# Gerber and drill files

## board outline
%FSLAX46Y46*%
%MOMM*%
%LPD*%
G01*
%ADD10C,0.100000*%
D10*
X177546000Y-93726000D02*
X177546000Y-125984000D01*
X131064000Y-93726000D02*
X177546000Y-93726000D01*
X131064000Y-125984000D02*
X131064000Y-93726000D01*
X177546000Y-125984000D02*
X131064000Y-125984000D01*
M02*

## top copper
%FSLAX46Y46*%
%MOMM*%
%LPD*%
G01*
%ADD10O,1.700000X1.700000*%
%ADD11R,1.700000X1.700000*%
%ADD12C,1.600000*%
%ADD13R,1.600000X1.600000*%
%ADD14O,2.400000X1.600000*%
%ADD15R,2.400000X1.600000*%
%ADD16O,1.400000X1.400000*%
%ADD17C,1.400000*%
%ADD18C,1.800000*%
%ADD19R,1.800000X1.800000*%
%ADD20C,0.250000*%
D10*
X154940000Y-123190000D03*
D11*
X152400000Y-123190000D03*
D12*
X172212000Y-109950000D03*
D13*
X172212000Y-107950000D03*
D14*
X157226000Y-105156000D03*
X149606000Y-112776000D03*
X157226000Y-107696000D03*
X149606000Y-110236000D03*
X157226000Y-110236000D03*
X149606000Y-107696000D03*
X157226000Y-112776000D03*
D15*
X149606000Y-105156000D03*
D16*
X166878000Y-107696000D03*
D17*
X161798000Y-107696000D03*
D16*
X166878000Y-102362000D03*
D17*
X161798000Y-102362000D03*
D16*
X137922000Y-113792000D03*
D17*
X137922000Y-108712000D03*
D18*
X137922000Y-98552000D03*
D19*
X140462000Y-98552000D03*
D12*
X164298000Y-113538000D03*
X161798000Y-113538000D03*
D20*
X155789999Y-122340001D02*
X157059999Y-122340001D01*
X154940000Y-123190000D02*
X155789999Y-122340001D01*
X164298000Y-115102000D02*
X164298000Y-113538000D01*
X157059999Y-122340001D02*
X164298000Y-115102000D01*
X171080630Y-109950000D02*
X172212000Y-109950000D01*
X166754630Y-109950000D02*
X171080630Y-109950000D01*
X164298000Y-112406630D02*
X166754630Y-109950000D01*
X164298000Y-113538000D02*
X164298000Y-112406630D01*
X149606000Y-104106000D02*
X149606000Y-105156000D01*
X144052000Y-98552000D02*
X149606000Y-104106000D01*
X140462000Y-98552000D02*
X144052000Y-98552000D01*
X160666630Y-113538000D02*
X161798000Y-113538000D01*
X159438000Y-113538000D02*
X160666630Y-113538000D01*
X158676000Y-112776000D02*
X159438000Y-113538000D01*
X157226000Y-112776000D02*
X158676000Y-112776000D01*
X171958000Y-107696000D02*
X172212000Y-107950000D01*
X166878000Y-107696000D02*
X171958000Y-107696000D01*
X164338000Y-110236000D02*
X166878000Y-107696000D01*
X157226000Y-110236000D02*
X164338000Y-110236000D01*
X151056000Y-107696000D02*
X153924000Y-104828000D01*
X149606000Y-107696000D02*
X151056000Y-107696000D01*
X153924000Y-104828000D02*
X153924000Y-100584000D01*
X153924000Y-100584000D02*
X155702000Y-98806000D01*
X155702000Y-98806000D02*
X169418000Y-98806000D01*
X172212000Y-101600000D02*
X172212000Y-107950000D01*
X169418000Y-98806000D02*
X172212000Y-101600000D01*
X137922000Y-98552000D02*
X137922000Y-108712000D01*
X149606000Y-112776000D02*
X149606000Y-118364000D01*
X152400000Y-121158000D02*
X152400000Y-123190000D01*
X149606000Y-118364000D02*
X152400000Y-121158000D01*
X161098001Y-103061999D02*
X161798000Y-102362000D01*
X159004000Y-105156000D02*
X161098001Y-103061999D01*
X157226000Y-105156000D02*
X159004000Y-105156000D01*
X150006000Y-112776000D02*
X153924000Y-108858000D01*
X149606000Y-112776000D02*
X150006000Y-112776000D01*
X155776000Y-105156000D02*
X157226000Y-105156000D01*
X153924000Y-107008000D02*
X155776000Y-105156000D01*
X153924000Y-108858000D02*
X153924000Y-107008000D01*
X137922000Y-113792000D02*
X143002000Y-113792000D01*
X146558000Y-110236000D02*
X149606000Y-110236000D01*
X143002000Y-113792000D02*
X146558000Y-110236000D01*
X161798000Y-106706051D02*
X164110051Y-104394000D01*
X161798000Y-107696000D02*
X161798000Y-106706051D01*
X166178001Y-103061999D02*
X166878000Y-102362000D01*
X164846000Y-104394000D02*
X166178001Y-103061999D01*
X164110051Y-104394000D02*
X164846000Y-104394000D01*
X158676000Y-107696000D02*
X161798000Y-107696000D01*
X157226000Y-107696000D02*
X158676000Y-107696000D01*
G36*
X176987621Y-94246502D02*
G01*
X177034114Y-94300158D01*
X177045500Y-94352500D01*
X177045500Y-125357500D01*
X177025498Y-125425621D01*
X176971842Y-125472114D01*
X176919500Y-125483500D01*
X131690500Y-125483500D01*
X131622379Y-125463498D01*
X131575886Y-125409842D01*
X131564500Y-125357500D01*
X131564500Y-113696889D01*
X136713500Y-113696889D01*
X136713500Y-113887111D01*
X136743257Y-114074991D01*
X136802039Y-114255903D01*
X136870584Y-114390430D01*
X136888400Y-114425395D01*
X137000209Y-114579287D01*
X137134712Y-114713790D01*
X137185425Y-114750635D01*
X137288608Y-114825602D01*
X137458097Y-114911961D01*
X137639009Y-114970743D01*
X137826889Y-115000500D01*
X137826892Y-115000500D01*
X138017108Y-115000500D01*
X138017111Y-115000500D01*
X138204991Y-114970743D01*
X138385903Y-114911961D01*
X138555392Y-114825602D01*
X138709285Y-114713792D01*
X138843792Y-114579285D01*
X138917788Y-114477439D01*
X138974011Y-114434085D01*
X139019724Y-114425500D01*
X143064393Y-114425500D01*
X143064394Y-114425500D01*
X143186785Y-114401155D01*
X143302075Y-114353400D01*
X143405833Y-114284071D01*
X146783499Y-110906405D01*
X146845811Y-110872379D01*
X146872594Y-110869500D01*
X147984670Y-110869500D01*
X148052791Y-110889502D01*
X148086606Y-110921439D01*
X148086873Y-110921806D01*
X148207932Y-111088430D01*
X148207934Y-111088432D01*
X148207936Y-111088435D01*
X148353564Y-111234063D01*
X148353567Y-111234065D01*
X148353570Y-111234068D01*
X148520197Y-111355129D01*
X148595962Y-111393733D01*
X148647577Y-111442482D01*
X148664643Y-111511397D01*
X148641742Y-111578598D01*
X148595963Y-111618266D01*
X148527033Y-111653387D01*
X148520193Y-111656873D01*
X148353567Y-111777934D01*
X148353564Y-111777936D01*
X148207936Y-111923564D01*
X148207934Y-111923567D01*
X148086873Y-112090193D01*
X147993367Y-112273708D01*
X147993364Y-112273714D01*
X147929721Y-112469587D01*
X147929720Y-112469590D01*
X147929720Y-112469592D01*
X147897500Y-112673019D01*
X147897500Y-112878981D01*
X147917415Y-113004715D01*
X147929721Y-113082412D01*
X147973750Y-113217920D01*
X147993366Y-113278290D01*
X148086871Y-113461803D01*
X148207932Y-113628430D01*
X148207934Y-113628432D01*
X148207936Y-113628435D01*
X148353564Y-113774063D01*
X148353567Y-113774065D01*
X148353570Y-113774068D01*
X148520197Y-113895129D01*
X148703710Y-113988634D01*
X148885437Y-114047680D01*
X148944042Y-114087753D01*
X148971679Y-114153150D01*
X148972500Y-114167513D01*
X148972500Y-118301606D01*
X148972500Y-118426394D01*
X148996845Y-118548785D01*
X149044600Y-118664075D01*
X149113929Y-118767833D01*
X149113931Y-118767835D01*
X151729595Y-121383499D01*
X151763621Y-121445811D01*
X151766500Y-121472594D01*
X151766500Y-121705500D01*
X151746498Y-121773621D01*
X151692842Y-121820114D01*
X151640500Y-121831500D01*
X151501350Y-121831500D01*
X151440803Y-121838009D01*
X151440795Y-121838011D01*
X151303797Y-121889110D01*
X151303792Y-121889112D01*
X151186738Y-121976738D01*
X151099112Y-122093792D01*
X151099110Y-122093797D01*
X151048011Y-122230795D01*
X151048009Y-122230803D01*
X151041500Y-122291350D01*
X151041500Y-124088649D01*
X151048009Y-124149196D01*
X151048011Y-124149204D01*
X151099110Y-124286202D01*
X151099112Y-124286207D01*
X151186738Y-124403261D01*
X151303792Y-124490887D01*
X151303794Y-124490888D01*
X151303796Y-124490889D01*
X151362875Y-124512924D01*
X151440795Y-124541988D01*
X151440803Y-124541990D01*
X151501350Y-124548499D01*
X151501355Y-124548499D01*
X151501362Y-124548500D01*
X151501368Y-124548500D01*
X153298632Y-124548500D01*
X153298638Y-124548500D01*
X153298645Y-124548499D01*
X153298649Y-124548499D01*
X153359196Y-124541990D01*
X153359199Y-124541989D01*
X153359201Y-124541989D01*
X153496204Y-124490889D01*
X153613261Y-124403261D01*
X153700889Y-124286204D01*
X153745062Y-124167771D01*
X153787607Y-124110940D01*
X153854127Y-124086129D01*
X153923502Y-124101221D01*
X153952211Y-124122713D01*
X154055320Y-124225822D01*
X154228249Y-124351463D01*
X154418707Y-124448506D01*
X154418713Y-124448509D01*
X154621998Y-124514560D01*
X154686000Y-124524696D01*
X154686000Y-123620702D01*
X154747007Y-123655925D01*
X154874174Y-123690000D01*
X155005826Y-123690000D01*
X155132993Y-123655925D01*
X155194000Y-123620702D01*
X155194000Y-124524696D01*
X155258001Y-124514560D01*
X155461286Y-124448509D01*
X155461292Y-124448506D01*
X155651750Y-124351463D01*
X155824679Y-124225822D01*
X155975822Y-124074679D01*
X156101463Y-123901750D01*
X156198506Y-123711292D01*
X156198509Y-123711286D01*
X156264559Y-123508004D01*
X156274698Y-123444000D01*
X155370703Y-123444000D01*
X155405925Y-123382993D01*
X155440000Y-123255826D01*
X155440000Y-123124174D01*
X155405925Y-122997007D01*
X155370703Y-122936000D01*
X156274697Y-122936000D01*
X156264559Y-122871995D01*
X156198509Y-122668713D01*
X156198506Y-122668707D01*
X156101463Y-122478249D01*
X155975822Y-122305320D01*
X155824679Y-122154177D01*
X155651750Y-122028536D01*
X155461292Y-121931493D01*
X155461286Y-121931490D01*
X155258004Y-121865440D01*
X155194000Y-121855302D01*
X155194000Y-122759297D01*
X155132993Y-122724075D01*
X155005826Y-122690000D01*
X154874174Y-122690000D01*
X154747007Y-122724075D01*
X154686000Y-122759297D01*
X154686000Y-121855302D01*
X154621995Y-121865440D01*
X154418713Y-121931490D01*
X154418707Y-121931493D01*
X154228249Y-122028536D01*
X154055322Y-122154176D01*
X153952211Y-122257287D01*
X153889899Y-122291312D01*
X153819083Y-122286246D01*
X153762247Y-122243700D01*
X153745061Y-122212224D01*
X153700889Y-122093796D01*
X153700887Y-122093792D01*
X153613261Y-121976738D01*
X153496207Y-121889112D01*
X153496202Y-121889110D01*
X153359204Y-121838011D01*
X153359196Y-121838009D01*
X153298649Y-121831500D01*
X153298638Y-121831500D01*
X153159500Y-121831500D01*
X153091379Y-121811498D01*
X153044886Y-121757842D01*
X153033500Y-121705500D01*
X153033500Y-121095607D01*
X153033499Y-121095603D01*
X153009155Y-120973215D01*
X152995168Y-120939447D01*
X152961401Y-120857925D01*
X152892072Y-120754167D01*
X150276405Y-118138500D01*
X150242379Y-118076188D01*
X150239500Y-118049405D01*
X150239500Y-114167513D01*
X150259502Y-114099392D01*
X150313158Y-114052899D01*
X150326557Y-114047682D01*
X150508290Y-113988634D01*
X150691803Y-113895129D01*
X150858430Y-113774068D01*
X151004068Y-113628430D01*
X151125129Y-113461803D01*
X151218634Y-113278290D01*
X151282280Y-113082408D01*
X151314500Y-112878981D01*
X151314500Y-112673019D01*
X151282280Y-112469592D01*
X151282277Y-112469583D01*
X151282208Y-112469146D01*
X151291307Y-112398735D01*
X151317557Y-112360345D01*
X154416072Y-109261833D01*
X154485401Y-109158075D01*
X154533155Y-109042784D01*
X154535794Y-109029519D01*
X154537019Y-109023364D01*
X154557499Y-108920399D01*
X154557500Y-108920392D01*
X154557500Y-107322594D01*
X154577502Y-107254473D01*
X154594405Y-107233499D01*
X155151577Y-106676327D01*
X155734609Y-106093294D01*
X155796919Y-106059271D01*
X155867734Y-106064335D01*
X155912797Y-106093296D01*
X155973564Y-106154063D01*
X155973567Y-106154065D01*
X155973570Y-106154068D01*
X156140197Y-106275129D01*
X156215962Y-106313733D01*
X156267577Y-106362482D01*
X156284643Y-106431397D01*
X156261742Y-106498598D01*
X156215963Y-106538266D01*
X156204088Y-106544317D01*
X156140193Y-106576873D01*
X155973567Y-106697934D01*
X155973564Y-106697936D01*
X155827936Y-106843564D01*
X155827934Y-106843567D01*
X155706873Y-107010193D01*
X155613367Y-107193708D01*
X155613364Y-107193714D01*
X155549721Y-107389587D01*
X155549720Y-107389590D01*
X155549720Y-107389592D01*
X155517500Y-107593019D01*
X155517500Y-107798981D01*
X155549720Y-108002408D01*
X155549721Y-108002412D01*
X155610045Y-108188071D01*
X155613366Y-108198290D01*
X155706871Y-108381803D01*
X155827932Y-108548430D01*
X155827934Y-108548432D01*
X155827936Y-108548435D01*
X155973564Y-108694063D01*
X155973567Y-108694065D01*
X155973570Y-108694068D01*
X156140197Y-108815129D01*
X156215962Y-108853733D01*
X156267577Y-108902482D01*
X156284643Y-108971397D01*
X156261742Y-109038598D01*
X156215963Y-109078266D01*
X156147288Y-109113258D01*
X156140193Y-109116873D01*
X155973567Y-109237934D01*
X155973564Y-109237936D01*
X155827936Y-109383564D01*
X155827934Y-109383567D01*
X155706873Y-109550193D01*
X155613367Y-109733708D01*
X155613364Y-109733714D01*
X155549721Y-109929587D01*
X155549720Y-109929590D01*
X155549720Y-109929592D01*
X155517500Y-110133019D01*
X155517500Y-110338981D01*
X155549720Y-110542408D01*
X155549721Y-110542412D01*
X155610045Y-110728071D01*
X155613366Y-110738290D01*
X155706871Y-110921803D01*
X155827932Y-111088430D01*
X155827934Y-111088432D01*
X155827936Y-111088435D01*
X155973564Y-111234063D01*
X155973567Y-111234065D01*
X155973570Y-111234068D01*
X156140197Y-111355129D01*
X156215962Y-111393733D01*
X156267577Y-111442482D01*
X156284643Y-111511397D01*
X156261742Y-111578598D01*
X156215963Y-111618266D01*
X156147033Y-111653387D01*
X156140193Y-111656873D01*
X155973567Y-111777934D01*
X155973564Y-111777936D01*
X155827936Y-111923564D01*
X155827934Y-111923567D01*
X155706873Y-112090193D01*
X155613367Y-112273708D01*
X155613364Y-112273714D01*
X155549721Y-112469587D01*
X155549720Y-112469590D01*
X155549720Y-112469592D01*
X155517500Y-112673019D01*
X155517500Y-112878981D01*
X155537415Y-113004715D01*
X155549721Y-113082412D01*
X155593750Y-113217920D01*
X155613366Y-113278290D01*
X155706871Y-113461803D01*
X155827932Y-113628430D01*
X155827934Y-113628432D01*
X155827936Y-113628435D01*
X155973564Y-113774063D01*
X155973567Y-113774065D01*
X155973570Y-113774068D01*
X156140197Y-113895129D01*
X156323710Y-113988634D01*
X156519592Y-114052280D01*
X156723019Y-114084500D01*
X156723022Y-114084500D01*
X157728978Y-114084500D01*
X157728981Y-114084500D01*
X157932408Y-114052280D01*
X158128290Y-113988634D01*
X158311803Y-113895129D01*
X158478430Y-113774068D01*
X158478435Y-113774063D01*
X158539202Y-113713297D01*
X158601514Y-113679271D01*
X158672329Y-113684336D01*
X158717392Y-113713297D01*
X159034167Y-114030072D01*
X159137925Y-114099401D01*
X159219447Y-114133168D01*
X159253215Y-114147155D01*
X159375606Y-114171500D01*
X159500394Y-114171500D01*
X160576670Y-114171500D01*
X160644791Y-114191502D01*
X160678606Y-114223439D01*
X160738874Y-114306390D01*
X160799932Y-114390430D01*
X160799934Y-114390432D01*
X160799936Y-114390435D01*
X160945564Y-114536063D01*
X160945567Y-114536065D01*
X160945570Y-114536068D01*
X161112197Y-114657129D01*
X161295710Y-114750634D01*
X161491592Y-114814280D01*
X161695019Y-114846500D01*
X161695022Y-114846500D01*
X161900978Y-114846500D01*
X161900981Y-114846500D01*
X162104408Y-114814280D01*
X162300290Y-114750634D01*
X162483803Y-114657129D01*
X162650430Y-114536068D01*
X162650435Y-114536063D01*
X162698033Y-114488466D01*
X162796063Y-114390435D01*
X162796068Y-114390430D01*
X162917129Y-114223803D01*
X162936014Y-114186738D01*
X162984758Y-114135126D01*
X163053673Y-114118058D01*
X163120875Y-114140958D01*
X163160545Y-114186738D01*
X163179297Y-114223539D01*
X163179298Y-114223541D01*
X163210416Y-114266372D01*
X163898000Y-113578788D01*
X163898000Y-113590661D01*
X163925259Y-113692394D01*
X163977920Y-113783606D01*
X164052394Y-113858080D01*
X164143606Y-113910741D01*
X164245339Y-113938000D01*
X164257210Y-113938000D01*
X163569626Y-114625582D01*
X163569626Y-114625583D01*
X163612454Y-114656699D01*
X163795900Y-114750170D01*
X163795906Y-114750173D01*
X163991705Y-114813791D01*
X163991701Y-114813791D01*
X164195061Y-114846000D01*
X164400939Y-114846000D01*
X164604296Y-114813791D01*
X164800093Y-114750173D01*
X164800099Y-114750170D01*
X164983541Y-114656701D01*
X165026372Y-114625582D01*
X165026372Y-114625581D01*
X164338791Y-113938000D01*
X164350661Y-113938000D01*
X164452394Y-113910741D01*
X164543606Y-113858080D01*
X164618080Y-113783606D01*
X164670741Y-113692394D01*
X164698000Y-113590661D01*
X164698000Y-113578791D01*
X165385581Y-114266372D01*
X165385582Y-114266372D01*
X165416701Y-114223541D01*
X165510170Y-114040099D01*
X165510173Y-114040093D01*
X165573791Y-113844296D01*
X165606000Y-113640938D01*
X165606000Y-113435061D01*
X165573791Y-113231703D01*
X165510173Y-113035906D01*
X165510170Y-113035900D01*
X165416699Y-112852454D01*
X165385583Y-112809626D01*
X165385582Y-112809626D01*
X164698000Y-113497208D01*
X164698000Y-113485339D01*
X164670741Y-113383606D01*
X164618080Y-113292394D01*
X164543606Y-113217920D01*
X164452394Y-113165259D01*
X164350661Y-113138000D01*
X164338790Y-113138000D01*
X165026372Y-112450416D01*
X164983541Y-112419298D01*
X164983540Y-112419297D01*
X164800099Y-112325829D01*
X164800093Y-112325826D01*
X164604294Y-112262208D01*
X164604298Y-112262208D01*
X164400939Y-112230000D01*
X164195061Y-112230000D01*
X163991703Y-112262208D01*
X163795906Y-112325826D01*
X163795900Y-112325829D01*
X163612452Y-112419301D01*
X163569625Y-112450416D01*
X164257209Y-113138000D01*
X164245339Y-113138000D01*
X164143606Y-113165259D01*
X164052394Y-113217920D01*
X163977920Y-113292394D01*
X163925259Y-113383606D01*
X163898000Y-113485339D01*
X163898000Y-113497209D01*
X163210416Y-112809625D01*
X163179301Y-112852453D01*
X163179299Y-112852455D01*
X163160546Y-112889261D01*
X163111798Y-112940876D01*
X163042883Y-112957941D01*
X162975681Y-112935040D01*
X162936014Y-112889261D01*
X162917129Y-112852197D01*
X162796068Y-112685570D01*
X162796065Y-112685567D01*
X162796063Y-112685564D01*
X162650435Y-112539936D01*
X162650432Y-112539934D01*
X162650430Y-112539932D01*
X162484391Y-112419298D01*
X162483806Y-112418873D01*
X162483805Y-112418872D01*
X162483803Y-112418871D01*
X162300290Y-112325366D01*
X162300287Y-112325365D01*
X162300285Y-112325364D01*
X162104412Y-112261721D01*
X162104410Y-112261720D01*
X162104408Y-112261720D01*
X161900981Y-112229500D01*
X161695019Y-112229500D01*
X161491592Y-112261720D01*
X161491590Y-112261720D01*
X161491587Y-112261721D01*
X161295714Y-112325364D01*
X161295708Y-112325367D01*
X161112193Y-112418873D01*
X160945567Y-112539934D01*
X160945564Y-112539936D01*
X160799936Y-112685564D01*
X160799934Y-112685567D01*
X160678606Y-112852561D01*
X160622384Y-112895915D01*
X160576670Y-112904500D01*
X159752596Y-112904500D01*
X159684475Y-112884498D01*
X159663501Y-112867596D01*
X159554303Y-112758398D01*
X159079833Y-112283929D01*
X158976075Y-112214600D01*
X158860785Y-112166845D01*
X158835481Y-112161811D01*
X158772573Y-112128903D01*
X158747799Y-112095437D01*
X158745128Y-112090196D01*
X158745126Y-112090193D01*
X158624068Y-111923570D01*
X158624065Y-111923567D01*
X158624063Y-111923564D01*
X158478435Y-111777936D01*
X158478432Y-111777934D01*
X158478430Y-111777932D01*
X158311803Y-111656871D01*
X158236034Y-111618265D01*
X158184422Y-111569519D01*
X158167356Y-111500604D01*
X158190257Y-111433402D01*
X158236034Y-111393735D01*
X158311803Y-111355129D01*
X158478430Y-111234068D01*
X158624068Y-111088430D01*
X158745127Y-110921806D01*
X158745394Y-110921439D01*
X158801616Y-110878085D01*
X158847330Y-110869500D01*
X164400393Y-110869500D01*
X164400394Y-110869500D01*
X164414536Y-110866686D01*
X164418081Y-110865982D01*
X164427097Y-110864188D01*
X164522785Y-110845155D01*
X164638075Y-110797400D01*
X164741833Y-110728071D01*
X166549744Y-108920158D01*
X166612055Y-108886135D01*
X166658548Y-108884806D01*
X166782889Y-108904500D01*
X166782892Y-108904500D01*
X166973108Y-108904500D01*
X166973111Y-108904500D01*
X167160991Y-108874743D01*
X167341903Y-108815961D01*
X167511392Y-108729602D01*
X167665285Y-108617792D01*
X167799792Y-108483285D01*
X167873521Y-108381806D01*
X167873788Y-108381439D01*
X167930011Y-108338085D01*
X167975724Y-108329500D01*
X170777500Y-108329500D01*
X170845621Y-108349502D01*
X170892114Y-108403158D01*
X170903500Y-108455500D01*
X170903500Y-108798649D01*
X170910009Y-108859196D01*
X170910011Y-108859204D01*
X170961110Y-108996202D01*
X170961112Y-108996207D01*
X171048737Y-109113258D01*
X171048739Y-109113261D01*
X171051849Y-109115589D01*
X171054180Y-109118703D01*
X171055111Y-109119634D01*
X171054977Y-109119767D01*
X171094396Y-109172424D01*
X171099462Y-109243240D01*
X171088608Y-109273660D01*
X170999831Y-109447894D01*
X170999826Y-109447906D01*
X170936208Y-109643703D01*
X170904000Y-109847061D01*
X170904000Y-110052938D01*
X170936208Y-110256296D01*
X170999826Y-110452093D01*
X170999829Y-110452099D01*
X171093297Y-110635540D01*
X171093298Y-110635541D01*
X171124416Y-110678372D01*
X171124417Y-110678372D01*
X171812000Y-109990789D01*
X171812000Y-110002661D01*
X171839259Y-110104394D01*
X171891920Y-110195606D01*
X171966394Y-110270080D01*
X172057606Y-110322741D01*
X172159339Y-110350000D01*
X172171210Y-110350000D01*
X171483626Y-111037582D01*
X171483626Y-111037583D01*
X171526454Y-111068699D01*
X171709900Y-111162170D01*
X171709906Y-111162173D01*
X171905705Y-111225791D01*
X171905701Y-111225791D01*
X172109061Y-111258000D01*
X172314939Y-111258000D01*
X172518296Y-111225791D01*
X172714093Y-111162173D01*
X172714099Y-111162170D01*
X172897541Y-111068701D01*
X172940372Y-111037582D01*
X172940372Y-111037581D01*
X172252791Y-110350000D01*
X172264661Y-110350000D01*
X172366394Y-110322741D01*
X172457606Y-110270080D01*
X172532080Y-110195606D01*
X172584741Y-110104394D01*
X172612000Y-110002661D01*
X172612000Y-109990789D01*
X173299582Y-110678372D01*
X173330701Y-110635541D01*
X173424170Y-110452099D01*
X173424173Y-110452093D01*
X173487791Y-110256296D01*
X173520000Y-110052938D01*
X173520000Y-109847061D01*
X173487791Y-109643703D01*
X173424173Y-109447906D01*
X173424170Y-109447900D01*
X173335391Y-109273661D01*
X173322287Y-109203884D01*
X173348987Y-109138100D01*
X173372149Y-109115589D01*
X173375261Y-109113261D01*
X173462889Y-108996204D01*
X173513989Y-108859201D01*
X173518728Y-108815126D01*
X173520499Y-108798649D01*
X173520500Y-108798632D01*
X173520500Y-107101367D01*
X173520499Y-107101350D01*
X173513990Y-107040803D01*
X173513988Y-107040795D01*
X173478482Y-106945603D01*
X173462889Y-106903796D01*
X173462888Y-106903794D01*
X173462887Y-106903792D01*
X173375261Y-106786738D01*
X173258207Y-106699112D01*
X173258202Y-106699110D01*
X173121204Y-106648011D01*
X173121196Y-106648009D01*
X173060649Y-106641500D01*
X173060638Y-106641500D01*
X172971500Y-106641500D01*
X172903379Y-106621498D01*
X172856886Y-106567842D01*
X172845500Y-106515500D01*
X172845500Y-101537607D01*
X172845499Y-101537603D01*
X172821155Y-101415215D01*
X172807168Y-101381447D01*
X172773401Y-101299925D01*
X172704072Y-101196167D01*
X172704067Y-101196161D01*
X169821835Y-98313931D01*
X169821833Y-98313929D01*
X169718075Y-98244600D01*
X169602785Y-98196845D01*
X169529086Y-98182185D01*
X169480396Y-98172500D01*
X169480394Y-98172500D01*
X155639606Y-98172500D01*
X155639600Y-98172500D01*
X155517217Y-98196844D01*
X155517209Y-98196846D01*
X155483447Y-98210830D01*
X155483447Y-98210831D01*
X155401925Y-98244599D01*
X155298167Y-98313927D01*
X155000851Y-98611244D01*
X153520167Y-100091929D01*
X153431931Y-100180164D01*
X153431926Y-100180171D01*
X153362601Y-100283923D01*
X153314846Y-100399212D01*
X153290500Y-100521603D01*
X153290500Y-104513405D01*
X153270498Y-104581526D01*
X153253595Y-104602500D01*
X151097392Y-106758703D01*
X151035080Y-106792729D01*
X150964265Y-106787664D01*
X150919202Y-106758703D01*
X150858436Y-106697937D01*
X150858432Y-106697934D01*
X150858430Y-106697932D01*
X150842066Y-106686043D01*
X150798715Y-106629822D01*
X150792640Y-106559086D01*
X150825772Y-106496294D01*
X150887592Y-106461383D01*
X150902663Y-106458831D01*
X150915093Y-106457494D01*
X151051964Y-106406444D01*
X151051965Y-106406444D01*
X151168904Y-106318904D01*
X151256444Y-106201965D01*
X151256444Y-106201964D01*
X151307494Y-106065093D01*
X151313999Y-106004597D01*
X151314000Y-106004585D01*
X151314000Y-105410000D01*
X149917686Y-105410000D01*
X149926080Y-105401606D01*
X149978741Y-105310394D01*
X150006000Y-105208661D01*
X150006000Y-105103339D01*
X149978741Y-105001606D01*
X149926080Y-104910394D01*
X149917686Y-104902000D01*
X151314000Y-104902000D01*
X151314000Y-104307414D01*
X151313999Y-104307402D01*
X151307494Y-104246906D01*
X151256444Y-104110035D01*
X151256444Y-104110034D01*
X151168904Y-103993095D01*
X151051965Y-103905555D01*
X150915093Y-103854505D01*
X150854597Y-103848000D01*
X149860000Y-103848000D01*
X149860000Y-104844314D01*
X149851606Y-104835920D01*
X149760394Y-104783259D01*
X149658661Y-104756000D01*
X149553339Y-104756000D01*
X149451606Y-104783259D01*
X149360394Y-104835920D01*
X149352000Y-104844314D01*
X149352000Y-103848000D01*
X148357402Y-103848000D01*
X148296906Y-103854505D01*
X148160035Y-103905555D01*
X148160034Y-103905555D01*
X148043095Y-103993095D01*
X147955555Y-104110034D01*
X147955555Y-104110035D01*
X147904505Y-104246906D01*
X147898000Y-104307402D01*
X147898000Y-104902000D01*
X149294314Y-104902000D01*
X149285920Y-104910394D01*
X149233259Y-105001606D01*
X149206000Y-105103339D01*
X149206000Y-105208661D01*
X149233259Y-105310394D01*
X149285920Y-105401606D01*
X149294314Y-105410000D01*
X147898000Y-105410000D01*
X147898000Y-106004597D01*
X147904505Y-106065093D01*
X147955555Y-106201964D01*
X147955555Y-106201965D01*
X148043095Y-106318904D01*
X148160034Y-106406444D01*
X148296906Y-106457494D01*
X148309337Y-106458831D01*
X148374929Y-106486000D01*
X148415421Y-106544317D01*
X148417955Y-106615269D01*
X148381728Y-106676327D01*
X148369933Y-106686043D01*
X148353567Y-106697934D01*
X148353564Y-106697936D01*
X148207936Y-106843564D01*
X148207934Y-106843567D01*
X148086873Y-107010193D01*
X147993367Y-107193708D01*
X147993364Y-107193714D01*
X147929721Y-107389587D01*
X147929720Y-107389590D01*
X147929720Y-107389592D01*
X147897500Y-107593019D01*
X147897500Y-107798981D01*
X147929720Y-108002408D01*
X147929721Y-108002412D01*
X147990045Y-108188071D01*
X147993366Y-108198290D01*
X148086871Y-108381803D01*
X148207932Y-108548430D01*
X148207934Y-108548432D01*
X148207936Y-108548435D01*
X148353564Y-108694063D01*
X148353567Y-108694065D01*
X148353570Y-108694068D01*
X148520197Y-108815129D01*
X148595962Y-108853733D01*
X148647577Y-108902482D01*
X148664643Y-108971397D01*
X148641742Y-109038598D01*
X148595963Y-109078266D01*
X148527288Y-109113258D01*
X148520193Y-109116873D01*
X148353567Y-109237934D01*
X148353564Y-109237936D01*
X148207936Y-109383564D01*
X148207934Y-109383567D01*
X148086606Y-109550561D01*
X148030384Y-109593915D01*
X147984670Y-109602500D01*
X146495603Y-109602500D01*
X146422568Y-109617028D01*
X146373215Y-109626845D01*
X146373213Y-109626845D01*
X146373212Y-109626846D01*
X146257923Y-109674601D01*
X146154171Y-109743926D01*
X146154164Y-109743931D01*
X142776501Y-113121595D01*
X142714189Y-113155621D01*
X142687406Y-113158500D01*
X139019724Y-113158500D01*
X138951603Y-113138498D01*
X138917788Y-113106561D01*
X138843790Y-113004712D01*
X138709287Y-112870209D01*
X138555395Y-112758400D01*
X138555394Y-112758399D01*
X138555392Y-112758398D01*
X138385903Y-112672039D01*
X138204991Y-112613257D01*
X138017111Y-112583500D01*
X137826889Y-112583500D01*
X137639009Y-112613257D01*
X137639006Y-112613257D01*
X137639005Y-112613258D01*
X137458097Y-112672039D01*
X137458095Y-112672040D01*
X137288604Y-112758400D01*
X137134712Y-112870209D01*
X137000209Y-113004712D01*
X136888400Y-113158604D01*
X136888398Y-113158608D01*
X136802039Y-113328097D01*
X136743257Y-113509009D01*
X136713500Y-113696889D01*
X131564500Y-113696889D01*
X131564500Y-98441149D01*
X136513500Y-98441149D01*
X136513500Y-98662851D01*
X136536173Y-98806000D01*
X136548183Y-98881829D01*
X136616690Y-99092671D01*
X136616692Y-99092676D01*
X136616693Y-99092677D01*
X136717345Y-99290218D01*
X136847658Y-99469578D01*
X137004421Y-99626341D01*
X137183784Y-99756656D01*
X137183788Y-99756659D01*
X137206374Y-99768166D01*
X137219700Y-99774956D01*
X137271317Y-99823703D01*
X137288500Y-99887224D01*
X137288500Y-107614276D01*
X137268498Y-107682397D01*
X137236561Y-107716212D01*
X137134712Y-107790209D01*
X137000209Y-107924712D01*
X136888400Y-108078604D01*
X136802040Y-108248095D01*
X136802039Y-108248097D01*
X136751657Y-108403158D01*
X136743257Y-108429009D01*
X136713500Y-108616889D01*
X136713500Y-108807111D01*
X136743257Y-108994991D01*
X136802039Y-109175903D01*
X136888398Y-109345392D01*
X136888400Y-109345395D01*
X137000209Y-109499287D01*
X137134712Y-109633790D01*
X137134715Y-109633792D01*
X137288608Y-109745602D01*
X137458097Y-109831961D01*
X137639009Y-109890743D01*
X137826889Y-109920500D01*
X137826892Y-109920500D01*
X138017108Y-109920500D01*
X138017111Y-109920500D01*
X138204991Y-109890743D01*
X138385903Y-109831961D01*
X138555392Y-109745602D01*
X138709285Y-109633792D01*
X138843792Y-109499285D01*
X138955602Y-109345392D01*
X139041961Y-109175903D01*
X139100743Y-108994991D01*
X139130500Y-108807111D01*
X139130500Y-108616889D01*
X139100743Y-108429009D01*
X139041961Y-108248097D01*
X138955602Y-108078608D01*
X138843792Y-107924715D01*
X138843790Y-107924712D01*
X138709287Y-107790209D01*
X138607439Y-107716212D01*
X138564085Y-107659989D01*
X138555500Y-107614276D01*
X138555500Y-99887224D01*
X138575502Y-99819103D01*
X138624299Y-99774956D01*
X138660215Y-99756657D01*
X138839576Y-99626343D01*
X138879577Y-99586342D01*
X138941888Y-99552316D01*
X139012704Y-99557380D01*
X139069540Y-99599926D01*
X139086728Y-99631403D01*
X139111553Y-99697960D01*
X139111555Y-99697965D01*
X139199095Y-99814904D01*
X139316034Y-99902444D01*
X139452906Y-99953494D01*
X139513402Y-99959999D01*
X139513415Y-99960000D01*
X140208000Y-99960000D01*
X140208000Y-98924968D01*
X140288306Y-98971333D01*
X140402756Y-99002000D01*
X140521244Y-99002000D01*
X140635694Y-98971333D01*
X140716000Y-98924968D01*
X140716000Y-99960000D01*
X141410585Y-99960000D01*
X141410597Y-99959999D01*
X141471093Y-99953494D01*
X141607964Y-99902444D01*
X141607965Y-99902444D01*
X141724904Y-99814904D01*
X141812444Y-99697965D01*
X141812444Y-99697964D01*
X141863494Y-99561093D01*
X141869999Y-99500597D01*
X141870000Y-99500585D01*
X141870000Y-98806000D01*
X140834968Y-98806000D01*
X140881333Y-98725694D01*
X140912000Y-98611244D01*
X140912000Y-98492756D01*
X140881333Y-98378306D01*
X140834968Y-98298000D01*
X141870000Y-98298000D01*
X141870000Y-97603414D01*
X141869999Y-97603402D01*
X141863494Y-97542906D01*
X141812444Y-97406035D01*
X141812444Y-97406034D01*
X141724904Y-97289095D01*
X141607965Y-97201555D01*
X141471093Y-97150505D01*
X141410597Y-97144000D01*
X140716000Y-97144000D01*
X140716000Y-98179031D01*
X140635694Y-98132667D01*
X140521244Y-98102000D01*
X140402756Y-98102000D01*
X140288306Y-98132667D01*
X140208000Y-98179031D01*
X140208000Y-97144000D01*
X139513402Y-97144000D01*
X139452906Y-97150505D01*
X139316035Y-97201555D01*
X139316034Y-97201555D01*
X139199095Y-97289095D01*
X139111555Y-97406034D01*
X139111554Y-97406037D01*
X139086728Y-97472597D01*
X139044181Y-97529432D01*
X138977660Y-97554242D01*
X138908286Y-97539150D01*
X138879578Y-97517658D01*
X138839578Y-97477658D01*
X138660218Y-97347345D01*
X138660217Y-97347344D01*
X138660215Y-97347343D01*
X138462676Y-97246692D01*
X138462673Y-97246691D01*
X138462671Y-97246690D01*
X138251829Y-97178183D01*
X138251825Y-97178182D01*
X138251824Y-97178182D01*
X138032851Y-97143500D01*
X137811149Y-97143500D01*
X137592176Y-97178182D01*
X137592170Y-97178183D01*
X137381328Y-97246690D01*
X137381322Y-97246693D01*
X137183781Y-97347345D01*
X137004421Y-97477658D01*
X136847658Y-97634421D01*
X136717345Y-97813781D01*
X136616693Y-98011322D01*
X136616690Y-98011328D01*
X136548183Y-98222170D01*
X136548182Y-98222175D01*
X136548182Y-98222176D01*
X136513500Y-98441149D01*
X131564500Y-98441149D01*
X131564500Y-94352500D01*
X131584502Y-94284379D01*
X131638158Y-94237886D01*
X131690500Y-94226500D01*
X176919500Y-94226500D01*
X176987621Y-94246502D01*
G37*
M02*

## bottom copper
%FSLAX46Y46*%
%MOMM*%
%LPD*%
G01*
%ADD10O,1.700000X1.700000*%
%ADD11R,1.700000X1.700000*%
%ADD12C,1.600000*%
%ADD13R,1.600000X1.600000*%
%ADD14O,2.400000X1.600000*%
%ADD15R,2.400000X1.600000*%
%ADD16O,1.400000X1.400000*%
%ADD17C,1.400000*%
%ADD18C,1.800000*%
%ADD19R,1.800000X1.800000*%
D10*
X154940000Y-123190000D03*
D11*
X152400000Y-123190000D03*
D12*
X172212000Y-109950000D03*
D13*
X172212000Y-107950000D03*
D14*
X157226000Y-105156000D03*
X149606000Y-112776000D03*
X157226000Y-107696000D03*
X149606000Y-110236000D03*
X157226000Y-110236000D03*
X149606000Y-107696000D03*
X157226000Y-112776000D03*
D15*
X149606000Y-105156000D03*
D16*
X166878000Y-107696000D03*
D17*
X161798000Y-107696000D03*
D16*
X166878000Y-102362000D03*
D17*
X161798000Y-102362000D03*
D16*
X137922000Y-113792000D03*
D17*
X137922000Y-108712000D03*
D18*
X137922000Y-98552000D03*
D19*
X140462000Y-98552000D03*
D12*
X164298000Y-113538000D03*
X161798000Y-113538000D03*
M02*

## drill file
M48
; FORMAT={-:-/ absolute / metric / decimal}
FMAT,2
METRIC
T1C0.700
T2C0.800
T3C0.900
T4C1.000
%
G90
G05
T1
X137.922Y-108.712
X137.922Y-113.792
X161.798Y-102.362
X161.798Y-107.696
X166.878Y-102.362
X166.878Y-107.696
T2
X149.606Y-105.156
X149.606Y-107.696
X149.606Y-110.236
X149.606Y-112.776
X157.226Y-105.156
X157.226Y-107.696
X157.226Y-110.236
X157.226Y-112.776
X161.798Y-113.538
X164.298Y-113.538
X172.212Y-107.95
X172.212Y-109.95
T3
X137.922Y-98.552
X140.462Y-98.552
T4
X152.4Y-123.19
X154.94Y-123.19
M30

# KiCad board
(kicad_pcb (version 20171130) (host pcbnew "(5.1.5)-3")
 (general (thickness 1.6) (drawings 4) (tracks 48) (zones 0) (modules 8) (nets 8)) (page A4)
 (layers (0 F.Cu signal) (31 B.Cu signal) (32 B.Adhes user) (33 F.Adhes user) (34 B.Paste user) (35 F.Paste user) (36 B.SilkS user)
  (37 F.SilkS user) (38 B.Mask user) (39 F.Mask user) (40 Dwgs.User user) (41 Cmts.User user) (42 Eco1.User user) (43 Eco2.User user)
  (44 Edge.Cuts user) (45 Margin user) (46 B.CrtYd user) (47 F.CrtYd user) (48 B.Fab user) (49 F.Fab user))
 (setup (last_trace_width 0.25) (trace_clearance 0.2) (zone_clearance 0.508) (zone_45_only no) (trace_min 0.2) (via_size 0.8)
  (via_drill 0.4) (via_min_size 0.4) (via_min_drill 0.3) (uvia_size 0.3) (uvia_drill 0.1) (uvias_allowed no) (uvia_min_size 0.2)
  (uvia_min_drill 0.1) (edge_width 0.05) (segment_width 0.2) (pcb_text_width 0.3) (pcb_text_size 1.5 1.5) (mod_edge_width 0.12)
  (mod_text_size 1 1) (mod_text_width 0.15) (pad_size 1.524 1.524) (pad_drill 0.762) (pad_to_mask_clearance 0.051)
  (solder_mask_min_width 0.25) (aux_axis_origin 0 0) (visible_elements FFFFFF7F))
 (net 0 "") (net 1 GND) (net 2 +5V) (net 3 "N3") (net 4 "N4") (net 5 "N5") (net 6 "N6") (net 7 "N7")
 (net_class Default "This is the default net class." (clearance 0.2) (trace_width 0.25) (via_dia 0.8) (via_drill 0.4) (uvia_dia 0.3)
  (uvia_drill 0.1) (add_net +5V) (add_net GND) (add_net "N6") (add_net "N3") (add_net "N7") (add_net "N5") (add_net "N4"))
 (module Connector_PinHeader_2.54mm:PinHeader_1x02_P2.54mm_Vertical (layer F.Cu) (at 152.4 123.19 90)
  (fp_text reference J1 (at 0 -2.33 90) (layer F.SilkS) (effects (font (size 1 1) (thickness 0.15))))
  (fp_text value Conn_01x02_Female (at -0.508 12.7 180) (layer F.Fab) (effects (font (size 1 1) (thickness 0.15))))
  (pad 2 thru_hole oval (at 0 2.54 90) (size 1.7 1.7) (drill 1) (layers *.Cu *.Mask) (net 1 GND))
  (pad 1 thru_hole rect (at 0 0 90) (size 1.7 1.7) (drill 1) (layers *.Cu *.Mask) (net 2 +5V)))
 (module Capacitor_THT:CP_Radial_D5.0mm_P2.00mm (layer F.Cu) (at 172.212 107.95 270)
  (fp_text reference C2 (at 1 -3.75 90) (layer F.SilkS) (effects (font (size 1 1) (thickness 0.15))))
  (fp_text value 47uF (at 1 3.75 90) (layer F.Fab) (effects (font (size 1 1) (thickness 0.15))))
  (pad 2 thru_hole circle (at 2 0 270) (size 1.6 1.6) (drill 0.8) (layers *.Cu *.Mask) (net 1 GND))
  (pad 1 thru_hole rect (at 0 0 270) (size 1.6 1.6) (drill 0.8) (layers *.Cu *.Mask) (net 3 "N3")))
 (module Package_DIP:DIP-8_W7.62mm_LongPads (layer F.Cu) (at 149.606 105.156)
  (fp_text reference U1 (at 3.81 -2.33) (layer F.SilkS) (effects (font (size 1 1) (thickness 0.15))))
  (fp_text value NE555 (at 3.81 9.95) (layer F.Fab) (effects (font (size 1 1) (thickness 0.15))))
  (pad 8 thru_hole oval (at 7.62 0) (size 2.4 1.6) (drill 0.8) (layers *.Cu *.Mask) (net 2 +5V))
  (pad 4 thru_hole oval (at 0 7.62) (size 2.4 1.6) (drill 0.8) (layers *.Cu *.Mask) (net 2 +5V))
  (pad 7 thru_hole oval (at 7.62 2.54) (size 2.4 1.6) (drill 0.8) (layers *.Cu *.Mask) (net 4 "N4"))
  (pad 3 thru_hole oval (at 0 5.08) (size 2.4 1.6) (drill 0.8) (layers *.Cu *.Mask) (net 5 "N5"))
  (pad 6 thru_hole oval (at 7.62 5.08) (size 2.4 1.6) (drill 0.8) (layers *.Cu *.Mask) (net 3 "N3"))
  (pad 2 thru_hole oval (at 0 2.54) (size 2.4 1.6) (drill 0.8) (layers *.Cu *.Mask) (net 3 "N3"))
  (pad 5 thru_hole oval (at 7.62 7.62) (size 2.4 1.6) (drill 0.8) (layers *.Cu *.Mask) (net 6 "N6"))
  (pad 1 thru_hole rect (at 0 0) (size 2.4 1.6) (drill 0.8) (layers *.Cu *.Mask) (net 1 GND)))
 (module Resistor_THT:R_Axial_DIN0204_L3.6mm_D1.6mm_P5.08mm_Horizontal (layer F.Cu) (at 161.798 107.696)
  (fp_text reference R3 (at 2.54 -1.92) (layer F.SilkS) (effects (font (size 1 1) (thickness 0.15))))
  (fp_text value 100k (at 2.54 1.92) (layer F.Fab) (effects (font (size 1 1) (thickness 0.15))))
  (pad 2 thru_hole oval (at 5.08 0) (size 1.4 1.4) (drill 0.7) (layers *.Cu *.Mask) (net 3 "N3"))
  (pad 1 thru_hole circle (at 0 0) (size 1.4 1.4) (drill 0.7) (layers *.Cu *.Mask) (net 4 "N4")))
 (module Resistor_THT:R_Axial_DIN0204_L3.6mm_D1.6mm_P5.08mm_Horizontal (layer F.Cu) (at 161.798 102.362)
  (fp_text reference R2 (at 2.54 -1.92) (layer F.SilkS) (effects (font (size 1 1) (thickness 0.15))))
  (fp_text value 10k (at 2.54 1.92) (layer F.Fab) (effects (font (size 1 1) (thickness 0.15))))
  (pad 2 thru_hole oval (at 5.08 0) (size 1.4 1.4) (drill 0.7) (layers *.Cu *.Mask) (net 4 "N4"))
  (pad 1 thru_hole circle (at 0 0) (size 1.4 1.4) (drill 0.7) (layers *.Cu *.Mask) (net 2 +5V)))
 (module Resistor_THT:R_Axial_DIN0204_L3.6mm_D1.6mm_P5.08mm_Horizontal (layer F.Cu) (at 137.922 108.712 270)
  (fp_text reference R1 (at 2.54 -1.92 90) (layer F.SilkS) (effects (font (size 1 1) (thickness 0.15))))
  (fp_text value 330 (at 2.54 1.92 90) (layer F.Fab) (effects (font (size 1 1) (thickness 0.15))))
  (pad 2 thru_hole oval (at 5.08 0 270) (size 1.4 1.4) (drill 0.7) (layers *.Cu *.Mask) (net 5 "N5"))
  (pad 1 thru_hole circle (at 0 0 270) (size 1.4 1.4) (drill 0.7) (layers *.Cu *.Mask) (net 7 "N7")))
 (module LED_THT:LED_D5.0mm (layer F.Cu) (at 140.462 98.552 180)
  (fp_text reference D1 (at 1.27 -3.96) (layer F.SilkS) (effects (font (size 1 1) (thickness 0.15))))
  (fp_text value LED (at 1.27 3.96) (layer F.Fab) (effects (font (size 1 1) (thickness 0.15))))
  (pad 2 thru_hole circle (at 2.54 0 180) (size 1.8 1.8) (drill 0.9) (layers *.Cu *.Mask) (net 7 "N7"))
  (pad 1 thru_hole rect (at 0 0 180) (size 1.8 1.8) (drill 0.9) (layers *.Cu *.Mask) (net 1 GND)))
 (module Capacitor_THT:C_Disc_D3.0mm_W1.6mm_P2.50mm (layer F.Cu) (at 161.798 113.538)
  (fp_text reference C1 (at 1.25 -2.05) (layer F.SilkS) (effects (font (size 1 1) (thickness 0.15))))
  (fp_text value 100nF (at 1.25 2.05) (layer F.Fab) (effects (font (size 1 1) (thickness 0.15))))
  (pad 2 thru_hole circle (at 2.5 0) (size 1.6 1.6) (drill 0.8) (layers *.Cu *.Mask) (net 1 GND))
  (pad 1 thru_hole circle (at 0 0) (size 1.6 1.6) (drill 0.8) (layers *.Cu *.Mask) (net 6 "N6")))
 (gr_line (start 177.546 93.726) (end 177.546 125.984) (layer Edge.Cuts) (width 0.1))
 (gr_line (start 131.064 93.726) (end 177.546 93.726) (layer Edge.Cuts) (width 0.1))
 (gr_line (start 131.064 125.984) (end 131.064 93.726) (layer Edge.Cuts) (width 0.1))
 (gr_line (start 177.546 125.984) (end 131.064 125.984) (layer Edge.Cuts) (width 0.1))
 (segment (start 155.789999 122.340001) (end 157.059999 122.340001) (width 0.25) (layer F.Cu) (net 1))
 (segment (start 154.94 123.19) (end 155.789999 122.340001) (width 0.25) (layer F.Cu) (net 1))
 (segment (start 164.298 115.102) (end 164.298 113.538) (width 0.25) (layer F.Cu) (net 1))
 (segment (start 157.059999 122.340001) (end 164.298 115.102) (width 0.25) (layer F.Cu) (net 1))
 (segment (start 171.08063 109.95) (end 172.212 109.95) (width 0.25) (layer F.Cu) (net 1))
 (segment (start 166.75463 109.95) (end 171.08063 109.95) (width 0.25) (layer F.Cu) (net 1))
 (segment (start 164.298 112.40663) (end 166.75463 109.95) (width 0.25) (layer F.Cu) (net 1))
 (segment (start 164.298 113.538) (end 164.298 112.40663) (width 0.25) (layer F.Cu) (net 1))
 (segment (start 149.606 104.106) (end 149.606 105.156) (width 0.25) (layer F.Cu) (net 1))
 (segment (start 144.052 98.552) (end 149.606 104.106) (width 0.25) (layer F.Cu) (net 1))
 (segment (start 140.462 98.552) (end 144.052 98.552) (width 0.25) (layer F.Cu) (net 1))
 (segment (start 160.66663 113.538) (end 161.798 113.538) (width 0.25) (layer F.Cu) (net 6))
 (segment (start 159.438 113.538) (end 160.66663 113.538) (width 0.25) (layer F.Cu) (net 6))
 (segment (start 158.676 112.776) (end 159.438 113.538) (width 0.25) (layer F.Cu) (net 6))
 (segment (start 157.226 112.776) (end 158.676 112.776) (width 0.25) (layer F.Cu) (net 6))
 (segment (start 171.958 107.696) (end 172.212 107.95) (width 0.25) (layer F.Cu) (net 3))
 (segment (start 166.878 107.696) (end 171.958 107.696) (width 0.25) (layer F.Cu) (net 3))
 (segment (start 164.338 110.236) (end 166.878 107.696) (width 0.25) (layer F.Cu) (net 3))
 (segment (start 157.226 110.236) (end 164.338 110.236) (width 0.25) (layer F.Cu) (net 3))
 (segment (start 151.056 107.696) (end 153.924 104.828) (width 0.25) (layer F.Cu) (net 3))
 (segment (start 149.606 107.696) (end 151.056 107.696) (width 0.25) (layer F.Cu) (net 3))
 (segment (start 153.924 104.828) (end 153.924 100.584) (width 0.25) (layer F.Cu) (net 3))
 (segment (start 153.924 100.584) (end 155.702 98.806) (width 0.25) (layer F.Cu) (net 3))
 (segment (start 155.702 98.806) (end 169.418 98.806) (width 0.25) (layer F.Cu) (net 3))
 (segment (start 172.212 101.6) (end 172.212 107.95) (width 0.25) (layer F.Cu) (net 3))
 (segment (start 169.418 98.806) (end 172.212 101.6) (width 0.25) (layer F.Cu) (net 3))
 (segment (start 137.922 98.552) (end 137.922 108.712) (width 0.25) (layer F.Cu) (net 7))
 (segment (start 149.606 112.776) (end 149.606 118.364) (width 0.25) (layer F.Cu) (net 2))
 (segment (start 152.4 121.158) (end 152.4 123.19) (width 0.25) (layer F.Cu) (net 2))
 (segment (start 149.606 118.364) (end 152.4 121.158) (width 0.25) (layer F.Cu) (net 2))
 (segment (start 161.098001 103.061999) (end 161.798 102.362) (width 0.25) (layer F.Cu) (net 2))
 (segment (start 159.004 105.156) (end 161.098001 103.061999) (width 0.25) (layer F.Cu) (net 2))
 (segment (start 157.226 105.156) (end 159.004 105.156) (width 0.25) (layer F.Cu) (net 2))
 (segment (start 150.006 112.776) (end 153.924 108.858) (width 0.25) (layer F.Cu) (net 2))
 (segment (start 149.606 112.776) (end 150.006 112.776) (width 0.25) (layer F.Cu) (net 2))
 (segment (start 155.776 105.156) (end 157.226 105.156) (width 0.25) (layer F.Cu) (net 2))
 (segment (start 153.924 107.008) (end 155.776 105.156) (width 0.25) (layer F.Cu) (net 2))
 (segment (start 153.924 108.858) (end 153.924 107.008) (width 0.25) (layer F.Cu) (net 2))
 (segment (start 137.922 113.792) (end 143.002 113.792) (width 0.25) (layer F.Cu) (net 5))
 (segment (start 146.558 110.236) (end 149.606 110.236) (width 0.25) (layer F.Cu) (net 5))
 (segment (start 143.002 113.792) (end 146.558 110.236) (width 0.25) (layer F.Cu) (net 5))
 (segment (start 161.798 106.706051) (end 164.110051 104.394) (width 0.25) (layer F.Cu) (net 4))
 (segment (start 161.798 107.696) (end 161.798 106.706051) (width 0.25) (layer F.Cu) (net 4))
 (segment (start 166.178001 103.061999) (end 166.878 102.362) (width 0.25) (layer F.Cu) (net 4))
 (segment (start 164.846 104.394) (end 166.178001 103.061999) (width 0.25) (layer F.Cu) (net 4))
 (segment (start 164.110051 104.394) (end 164.846 104.394) (width 0.25) (layer F.Cu) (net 4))
 (segment (start 158.676 107.696) (end 161.798 107.696) (width 0.25) (layer F.Cu) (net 4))
 (segment (start 157.226 107.696) (end 158.676 107.696) (width 0.25) (layer F.Cu) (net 4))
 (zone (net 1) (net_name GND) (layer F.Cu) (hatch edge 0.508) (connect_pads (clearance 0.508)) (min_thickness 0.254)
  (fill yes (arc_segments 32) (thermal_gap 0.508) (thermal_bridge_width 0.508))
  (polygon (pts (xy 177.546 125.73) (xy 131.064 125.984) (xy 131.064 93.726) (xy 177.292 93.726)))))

